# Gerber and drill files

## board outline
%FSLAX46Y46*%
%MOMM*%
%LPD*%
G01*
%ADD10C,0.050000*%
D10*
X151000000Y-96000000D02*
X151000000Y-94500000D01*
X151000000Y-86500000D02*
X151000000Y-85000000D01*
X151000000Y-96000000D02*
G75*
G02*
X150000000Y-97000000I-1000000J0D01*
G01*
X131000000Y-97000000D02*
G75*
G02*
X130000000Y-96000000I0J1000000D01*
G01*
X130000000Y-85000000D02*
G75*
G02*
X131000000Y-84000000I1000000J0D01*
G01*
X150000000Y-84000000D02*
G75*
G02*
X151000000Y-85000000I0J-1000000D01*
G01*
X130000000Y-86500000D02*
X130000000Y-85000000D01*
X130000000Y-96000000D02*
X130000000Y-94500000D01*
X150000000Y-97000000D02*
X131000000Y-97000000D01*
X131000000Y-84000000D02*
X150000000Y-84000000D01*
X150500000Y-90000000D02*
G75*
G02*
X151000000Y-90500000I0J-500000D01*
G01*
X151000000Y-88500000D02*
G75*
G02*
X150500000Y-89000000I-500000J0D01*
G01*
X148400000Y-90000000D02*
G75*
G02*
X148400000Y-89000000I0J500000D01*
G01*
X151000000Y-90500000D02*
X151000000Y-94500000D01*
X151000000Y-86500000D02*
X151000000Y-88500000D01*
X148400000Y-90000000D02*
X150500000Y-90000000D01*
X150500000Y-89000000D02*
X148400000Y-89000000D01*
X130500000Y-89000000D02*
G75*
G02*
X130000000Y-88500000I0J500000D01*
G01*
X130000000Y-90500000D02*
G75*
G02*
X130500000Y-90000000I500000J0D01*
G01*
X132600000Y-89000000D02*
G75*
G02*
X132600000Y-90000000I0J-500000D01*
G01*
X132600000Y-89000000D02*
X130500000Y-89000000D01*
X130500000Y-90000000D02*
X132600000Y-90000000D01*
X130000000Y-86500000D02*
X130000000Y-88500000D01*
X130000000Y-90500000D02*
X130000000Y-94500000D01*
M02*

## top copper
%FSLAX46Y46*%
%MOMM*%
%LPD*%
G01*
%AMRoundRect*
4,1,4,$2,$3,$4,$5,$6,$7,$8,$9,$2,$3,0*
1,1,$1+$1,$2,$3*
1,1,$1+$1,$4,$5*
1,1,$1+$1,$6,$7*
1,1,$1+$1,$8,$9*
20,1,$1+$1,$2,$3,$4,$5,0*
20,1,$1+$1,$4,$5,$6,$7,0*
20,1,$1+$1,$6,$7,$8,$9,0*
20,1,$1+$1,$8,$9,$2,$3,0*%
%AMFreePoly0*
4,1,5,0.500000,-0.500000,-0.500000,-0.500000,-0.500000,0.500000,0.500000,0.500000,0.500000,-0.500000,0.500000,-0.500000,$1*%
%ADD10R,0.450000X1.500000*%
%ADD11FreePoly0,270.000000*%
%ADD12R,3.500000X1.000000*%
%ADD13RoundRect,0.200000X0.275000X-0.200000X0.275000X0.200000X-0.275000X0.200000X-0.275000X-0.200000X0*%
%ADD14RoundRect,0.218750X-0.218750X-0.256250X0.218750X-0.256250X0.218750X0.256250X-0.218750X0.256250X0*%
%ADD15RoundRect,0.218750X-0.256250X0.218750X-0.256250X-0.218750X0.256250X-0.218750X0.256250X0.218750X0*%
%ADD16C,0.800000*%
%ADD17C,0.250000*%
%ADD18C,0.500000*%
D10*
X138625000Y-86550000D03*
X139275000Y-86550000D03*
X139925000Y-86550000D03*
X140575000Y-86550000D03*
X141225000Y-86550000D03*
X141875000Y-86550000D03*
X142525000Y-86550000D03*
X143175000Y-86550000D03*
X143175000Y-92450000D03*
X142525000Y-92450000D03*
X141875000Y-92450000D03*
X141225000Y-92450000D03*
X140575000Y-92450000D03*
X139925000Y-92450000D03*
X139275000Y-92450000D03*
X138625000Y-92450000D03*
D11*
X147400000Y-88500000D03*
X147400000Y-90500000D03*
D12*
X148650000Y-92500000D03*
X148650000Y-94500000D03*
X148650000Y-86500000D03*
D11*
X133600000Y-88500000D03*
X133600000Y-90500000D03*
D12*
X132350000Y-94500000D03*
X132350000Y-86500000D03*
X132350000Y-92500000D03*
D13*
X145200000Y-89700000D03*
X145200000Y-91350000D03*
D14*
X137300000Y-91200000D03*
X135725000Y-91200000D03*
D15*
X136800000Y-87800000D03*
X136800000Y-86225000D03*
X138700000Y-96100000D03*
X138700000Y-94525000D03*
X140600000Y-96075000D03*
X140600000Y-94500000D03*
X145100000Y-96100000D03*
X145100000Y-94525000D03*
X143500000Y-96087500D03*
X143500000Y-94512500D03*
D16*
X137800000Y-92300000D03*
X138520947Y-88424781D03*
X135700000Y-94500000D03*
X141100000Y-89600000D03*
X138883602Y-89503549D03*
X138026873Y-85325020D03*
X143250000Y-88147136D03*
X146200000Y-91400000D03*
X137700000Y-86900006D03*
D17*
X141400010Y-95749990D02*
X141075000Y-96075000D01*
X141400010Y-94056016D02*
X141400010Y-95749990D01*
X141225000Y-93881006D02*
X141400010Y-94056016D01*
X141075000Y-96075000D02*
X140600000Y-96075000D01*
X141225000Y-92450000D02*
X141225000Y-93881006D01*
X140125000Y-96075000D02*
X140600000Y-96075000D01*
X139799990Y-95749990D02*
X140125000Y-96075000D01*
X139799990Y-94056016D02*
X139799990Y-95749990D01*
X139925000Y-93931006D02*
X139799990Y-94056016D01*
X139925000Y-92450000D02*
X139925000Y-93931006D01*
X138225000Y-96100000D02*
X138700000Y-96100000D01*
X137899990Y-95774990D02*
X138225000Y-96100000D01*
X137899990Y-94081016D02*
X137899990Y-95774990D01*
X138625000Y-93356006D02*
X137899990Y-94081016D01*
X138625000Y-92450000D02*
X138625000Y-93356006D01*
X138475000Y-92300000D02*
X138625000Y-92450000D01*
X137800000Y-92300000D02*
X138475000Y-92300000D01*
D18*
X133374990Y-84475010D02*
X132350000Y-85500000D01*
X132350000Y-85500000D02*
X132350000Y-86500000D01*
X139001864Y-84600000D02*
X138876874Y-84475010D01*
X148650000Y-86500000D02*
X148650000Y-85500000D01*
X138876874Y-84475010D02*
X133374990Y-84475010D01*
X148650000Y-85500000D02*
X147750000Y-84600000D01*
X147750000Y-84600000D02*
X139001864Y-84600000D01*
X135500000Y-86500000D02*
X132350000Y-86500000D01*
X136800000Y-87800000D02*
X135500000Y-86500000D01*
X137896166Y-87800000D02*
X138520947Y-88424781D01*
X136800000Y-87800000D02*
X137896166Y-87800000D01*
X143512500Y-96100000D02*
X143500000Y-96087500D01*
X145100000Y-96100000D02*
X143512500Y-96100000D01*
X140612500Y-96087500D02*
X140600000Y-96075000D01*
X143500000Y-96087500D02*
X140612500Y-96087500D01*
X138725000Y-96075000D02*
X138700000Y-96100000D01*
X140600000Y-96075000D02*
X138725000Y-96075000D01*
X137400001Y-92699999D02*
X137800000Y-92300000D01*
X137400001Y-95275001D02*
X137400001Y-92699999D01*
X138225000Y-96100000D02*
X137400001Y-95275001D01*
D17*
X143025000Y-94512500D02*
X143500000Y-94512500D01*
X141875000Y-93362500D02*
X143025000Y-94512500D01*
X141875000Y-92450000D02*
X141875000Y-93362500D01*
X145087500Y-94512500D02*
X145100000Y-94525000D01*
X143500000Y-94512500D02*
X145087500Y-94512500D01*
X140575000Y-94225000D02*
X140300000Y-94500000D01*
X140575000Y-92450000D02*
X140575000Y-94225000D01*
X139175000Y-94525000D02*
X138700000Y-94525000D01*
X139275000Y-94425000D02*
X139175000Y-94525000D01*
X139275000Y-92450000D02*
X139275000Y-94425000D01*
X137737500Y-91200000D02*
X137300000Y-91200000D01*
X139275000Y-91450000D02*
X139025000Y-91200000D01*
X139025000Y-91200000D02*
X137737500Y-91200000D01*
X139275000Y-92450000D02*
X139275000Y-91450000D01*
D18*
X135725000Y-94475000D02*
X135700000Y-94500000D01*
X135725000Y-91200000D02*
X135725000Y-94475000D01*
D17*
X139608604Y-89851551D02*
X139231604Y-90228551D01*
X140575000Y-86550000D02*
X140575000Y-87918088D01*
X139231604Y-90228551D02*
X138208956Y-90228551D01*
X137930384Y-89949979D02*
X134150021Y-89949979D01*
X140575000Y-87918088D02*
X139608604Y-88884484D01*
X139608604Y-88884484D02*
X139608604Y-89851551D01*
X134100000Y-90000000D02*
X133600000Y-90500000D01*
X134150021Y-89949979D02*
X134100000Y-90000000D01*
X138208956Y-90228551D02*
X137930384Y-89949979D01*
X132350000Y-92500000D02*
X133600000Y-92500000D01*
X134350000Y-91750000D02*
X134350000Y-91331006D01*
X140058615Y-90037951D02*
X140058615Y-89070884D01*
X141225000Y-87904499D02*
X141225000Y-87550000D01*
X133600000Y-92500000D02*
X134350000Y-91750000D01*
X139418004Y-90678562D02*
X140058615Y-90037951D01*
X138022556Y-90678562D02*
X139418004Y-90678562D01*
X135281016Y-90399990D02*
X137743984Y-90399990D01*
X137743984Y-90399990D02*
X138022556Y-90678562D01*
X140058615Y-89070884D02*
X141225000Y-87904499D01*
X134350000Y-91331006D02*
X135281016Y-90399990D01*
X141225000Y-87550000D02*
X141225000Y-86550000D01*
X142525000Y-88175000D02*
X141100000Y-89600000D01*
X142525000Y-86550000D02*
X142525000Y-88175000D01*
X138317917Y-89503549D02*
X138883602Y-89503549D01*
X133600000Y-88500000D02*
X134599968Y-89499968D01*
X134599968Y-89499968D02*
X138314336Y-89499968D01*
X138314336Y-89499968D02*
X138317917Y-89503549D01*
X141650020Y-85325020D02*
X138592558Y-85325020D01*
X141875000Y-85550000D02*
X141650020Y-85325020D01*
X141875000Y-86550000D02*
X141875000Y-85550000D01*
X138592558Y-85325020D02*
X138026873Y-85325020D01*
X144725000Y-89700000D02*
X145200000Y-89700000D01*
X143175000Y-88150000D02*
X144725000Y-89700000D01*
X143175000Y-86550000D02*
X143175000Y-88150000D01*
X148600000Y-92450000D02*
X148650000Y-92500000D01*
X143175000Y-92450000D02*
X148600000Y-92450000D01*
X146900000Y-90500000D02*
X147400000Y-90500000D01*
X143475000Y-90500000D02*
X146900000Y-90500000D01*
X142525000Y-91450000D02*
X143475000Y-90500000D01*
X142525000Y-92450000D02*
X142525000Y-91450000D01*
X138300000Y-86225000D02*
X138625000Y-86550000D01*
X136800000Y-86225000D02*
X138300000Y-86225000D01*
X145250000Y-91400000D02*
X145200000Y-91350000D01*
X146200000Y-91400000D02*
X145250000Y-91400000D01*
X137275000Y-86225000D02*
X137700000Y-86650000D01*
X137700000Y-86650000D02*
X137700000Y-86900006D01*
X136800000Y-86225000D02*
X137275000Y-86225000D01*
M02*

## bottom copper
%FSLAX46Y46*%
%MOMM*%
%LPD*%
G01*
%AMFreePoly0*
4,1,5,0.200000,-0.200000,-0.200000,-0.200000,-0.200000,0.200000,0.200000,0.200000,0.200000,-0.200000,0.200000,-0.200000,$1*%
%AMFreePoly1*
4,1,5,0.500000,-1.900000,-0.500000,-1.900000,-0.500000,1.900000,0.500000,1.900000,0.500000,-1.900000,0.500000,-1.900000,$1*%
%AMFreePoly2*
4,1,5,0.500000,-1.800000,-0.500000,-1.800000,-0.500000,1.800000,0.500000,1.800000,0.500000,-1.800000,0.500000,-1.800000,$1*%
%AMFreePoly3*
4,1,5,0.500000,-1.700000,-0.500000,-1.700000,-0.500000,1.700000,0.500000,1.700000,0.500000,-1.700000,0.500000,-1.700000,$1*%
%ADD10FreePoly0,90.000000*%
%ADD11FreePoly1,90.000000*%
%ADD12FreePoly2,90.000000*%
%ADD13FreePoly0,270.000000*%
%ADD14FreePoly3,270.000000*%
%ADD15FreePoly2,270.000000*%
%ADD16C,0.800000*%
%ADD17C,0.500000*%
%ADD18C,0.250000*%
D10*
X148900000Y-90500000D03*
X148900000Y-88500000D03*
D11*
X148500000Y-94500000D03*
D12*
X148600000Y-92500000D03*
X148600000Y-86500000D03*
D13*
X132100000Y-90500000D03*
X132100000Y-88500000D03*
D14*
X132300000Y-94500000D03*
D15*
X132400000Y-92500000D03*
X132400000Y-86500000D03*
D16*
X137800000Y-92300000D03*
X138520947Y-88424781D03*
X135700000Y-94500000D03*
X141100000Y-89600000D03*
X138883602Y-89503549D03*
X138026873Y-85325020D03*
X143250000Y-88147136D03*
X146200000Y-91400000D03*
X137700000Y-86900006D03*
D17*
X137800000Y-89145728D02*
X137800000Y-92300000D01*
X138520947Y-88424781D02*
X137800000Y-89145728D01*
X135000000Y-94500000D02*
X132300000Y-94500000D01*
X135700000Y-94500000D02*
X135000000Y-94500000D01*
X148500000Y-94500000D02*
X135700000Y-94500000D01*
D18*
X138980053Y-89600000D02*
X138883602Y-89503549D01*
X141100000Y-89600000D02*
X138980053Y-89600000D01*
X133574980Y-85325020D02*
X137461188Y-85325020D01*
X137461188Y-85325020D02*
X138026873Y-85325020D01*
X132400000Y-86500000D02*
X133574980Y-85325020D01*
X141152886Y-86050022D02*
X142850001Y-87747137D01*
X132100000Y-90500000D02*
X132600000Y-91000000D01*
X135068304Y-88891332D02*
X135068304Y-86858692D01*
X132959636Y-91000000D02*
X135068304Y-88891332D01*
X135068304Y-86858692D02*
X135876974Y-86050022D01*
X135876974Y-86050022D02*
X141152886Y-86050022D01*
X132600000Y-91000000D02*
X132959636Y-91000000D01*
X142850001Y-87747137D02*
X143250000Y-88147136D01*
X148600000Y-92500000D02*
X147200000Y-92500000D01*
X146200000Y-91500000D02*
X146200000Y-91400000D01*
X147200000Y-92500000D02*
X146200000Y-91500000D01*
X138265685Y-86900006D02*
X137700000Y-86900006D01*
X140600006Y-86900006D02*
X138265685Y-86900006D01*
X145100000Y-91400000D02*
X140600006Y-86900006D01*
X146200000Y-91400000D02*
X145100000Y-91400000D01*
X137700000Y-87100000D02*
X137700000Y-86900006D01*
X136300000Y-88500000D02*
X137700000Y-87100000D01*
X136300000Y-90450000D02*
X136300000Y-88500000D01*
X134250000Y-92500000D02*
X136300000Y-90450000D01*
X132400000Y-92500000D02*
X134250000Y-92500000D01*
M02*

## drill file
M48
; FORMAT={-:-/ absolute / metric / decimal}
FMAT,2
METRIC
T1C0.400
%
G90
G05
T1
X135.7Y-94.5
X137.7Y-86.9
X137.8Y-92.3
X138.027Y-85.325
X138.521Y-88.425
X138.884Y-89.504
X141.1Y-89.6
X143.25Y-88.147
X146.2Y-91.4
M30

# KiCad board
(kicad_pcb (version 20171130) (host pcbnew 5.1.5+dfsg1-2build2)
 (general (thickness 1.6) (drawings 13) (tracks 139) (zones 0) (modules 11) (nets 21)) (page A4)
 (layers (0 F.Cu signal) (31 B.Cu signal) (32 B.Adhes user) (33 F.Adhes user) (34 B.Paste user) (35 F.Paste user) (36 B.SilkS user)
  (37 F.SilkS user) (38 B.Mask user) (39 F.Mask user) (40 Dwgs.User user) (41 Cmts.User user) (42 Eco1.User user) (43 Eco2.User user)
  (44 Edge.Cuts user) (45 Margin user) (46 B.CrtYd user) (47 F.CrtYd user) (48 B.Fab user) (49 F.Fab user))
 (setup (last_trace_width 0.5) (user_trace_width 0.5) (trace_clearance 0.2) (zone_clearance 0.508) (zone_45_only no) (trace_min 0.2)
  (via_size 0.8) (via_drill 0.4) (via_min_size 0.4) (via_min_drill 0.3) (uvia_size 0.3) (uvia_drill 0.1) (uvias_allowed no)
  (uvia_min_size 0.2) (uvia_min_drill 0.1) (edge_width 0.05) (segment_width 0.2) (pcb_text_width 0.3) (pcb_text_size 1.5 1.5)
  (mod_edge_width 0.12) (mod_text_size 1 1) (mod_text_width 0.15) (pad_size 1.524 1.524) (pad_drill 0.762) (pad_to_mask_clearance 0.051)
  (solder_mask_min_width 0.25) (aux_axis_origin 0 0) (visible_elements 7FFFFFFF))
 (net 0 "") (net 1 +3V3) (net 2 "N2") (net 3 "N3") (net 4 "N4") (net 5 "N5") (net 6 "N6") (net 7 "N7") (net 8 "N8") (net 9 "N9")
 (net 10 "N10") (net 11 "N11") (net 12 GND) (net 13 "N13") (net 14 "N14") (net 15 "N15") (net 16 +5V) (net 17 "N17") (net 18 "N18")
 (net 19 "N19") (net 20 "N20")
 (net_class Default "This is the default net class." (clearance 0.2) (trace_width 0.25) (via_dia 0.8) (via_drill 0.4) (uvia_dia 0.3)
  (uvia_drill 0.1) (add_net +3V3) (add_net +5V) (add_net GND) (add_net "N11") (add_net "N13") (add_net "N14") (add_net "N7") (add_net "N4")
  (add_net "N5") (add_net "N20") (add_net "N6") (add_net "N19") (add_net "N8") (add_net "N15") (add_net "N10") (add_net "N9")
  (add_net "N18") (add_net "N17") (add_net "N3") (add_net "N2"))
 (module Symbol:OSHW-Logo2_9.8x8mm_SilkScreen (layer B.Cu) (at 141 90 180)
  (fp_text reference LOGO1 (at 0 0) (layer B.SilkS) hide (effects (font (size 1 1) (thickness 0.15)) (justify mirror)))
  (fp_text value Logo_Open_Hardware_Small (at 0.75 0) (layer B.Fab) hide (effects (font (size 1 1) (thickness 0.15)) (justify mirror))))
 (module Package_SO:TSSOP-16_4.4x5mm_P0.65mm (layer F.Cu) (at 140.9 89.5 90)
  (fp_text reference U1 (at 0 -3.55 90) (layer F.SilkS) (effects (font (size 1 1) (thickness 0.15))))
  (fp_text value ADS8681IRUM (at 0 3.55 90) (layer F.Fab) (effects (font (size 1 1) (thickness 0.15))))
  (pad 16 smd rect (at 2.95 -2.275 90) (size 1.5 0.45) (layers F.Cu F.Paste F.Mask) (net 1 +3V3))
  (pad 15 smd rect (at 2.95 -1.625 90) (size 1.5 0.45) (layers F.Cu F.Paste F.Mask) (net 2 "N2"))
  (pad 14 smd rect (at 2.95 -0.975 90) (size 1.5 0.45) (layers F.Cu F.Paste F.Mask) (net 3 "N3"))
  (pad 13 smd rect (at 2.95 -0.325 90) (size 1.5 0.45) (layers F.Cu F.Paste F.Mask) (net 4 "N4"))
  (pad 12 smd rect (at 2.95 0.325 90) (size 1.5 0.45) (layers F.Cu F.Paste F.Mask) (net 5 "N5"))
  (pad 11 smd rect (at 2.95 0.975 90) (size 1.5 0.45) (layers F.Cu F.Paste F.Mask) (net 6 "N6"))
  (pad 10 smd rect (at 2.95 1.625 90) (size 1.5 0.45) (layers F.Cu F.Paste F.Mask) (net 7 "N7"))
  (pad 9 smd rect (at 2.95 2.275 90) (size 1.5 0.45) (layers F.Cu F.Paste F.Mask) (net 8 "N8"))
  (pad 8 smd rect (at -2.95 2.275 90) (size 1.5 0.45) (layers F.Cu F.Paste F.Mask) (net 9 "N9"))
  (pad 7 smd rect (at -2.95 1.625 90) (size 1.5 0.45) (layers F.Cu F.Paste F.Mask) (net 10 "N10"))
  (pad 6 smd rect (at -2.95 0.975 90) (size 1.5 0.45) (layers F.Cu F.Paste F.Mask) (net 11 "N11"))
  (pad 5 smd rect (at -2.95 0.325 90) (size 1.5 0.45) (layers F.Cu F.Paste F.Mask) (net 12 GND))
  (pad 4 smd rect (at -2.95 -0.325 90) (size 1.5 0.45) (layers F.Cu F.Paste F.Mask) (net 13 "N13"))
  (pad 3 smd rect (at -2.95 -0.975 90) (size 1.5 0.45) (layers F.Cu F.Paste F.Mask) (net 12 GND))
  (pad 2 smd rect (at -2.95 -1.625 90) (size 1.5 0.45) (layers F.Cu F.Paste F.Mask) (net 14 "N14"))
  (pad 1 smd rect (at -2.95 -2.275 90) (size 1.5 0.45) (layers F.Cu F.Paste F.Mask) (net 12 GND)))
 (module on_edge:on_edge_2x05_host (layer F.Cu) (at 151 90.5 270)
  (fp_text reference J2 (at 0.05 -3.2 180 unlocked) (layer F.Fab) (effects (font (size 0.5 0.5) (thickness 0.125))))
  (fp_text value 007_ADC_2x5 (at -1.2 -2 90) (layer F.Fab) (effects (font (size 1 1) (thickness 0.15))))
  (fp_arc (start 0 0.5) (end 0 0) (angle -90) (layer Edge.Cuts) (width 0.05))
  (fp_arc (start -2 0.5) (end -1.5 0.5) (angle -90) (layer Edge.Cuts) (width 0.05))
  (fp_arc (start -1 2.6) (end -1.5 2.6) (angle -180) (layer Edge.Cuts) (width 0.05))
  (fp_line (start 0 0) (end 4 0) (layer Edge.Cuts) (width 0.05))
  (fp_line (start -4 0) (end -2 0) (layer Edge.Cuts) (width 0.05))
  (fp_line (start -0.5 2.6) (end -0.5 0.5) (layer Edge.Cuts) (width 0.05))
  (fp_line (start -1.5 0.5) (end -1.5 2.6) (layer Edge.Cuts) (width 0.05))
  (pad 2 smd custom (at -2 3.6 270) (size 1 1) (layers F.Cu F.Mask) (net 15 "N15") (zone_connect 0)
   (options (clearance outline) (anchor rect)) (primitives))
  (pad 3 smd custom (at 0 3.6 270) (size 1 1) (layers F.Cu F.Mask) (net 10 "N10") (zone_connect 0)
   (options (clearance outline) (anchor rect)) (primitives))
  (pad 8 smd custom (at 0 2.1 90) (size 0.4 0.4) (layers B.Cu B.Mask) (zone_connect 0) (options (clearance outline) (anchor rect))
   (primitives))
  (pad 7 smd custom (at -2 2.1 90) (size 0.4 0.4) (layers B.Cu B.Mask) (zone_connect 0) (options (clearance outline) (anchor rect))
   (primitives))
  (pad 4 smd rect (at 2 2.35 270) (size 1 3.5) (layers F.Cu F.Mask) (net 9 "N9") (zone_connect 0))
  (pad 10 smd custom (at 4 2.5 90) (size 1 3.8) (layers B.Cu B.Mask) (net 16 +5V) (zone_connect 0)
   (options (clearance outline) (anchor rect)) (primitives))
  (pad 9 smd custom (at 2 2.4 90) (size 1 3.6) (layers B.Cu B.Mask) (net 1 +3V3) (zone_connect 0)
   (options (clearance outline) (anchor rect)) (primitives))
  (pad 6 smd custom (at -4 2.4 90) (size 1 3.6) (layers B.Cu B.Mask) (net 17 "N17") (zone_connect 0)
   (options (clearance outline) (anchor rect)) (primitives))
  (pad 5 smd rect (at 4 2.35 270) (size 1 3.5) (layers F.Cu F.Mask) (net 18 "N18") (zone_connect 0))
  (pad 1 smd rect (at -4 2.35 270) (size 1 3.5) (layers F.Cu F.Mask) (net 12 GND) (zone_connect 0)))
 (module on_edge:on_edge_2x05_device (layer F.Cu) (at 130 90.5 270)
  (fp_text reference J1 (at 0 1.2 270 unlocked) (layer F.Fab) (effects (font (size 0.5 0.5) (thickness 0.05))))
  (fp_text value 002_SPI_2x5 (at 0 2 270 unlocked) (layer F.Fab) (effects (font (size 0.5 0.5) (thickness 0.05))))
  (fp_arc (start -2 -0.5) (end -2 0) (angle -90) (layer Edge.Cuts) (width 0.05))
  (fp_arc (start 0 -0.5) (end -0.5 -0.5) (angle -90) (layer Edge.Cuts) (width 0.05))
  (fp_arc (start -1 -2.6) (end -0.5 -2.6) (angle -180) (layer Edge.Cuts) (width 0.05))
  (fp_line (start -1.5 -2.6) (end -1.5 -0.5) (layer Edge.Cuts) (width 0.05))
  (fp_line (start -0.5 -0.5) (end -0.5 -2.6) (layer Edge.Cuts) (width 0.05))
  (fp_line (start -4 0) (end -2 0) (layer Edge.Cuts) (width 0.05))
  (fp_line (start 0 0) (end 4 0) (layer Edge.Cuts) (width 0.05))
  (pad 2 smd custom (at -2 -3.6 270) (size 1 1) (layers F.Cu F.Mask) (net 7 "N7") (zone_connect 0)
   (options (clearance outline) (anchor rect)) (primitives))
  (pad 3 smd custom (at 0 -3.6 270) (size 1 1) (layers F.Cu F.Mask) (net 4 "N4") (zone_connect 0)
   (options (clearance outline) (anchor rect)) (primitives))
  (pad 8 smd custom (at 0 -2.1 270) (size 0.4 0.4) (layers B.Cu B.Mask) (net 8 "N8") (zone_connect 0)
   (options (clearance outline) (anchor rect)) (primitives))
  (pad 7 smd custom (at -2 -2.1 270) (size 0.4 0.4) (layers B.Cu B.Mask) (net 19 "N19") (zone_connect 0)
   (options (clearance outline) (anchor rect)) (primitives))
  (pad 10 smd custom (at 4 -2.3 270) (size 1 3.4) (layers B.Cu B.Mask) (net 16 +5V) (zone_connect 0)
   (options (clearance outline) (anchor rect)) (primitives))
  (pad 9 smd custom (at 2 -2.4 270) (size 1 3.6) (layers B.Cu B.Mask) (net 1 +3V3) (zone_connect 0)
   (options (clearance outline) (anchor rect)) (primitives))
  (pad 6 smd custom (at -4 -2.4 270) (size 1 3.6) (layers B.Cu B.Mask) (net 6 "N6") (zone_connect 0)
   (options (clearance outline) (anchor rect)) (primitives))
  (pad 5 smd rect (at 4 -2.35 90) (size 1 3.5) (layers F.Cu F.Mask) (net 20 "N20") (zone_connect 0))
  (pad 1 smd rect (at -4 -2.35 90) (size 1 3.5) (layers F.Cu F.Mask) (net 12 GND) (zone_connect 0))
  (pad 4 smd rect (at 2 -2.35 90) (size 1 3.5) (layers F.Cu F.Mask) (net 5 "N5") (zone_connect 0)))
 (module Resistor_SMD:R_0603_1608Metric (layer F.Cu) (at 145.2 90.525 90)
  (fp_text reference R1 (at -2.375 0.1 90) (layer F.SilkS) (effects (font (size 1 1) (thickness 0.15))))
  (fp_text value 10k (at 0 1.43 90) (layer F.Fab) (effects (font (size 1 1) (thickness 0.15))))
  (pad 2 smd roundrect (at 0.825 0 90) (size 0.8 0.95) (layers F.Cu F.Paste F.Mask) (roundrect_rratio 0.25) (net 8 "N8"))
  (pad 1 smd roundrect (at -0.825 0 90) (size 0.8 0.95) (layers F.Cu F.Paste F.Mask) (roundrect_rratio 0.25) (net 1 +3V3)))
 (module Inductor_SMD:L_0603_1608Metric (layer F.Cu) (at 136.5125 91.2)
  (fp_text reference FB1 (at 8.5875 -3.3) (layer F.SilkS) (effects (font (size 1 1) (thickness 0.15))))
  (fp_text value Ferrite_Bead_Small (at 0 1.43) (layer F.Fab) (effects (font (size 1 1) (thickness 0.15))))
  (pad 2 smd roundrect (at 0.7875 0) (size 0.875 0.95) (layers F.Cu F.Paste F.Mask) (roundrect_rratio 0.25) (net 14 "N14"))
  (pad 1 smd roundrect (at -0.7875 0) (size 0.875 0.95) (layers F.Cu F.Paste F.Mask) (roundrect_rratio 0.25) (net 16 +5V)))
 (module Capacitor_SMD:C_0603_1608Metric (layer F.Cu) (at 136.8 87.0125 270)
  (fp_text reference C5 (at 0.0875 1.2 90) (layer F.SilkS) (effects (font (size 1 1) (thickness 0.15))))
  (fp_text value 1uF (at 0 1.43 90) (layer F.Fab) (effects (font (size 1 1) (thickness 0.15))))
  (pad 2 smd roundrect (at 0.7875 0 270) (size 0.875 0.95) (layers F.Cu F.Paste F.Mask) (roundrect_rratio 0.25) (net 12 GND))
  (pad 1 smd roundrect (at -0.7875 0 270) (size 0.875 0.95) (layers F.Cu F.Paste F.Mask) (roundrect_rratio 0.25) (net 1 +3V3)))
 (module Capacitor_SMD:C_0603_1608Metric (layer F.Cu) (at 138.7 95.3125 270)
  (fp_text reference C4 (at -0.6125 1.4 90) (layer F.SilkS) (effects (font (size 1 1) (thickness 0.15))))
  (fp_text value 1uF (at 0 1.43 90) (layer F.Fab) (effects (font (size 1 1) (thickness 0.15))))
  (pad 2 smd roundrect (at 0.7875 0 270) (size 0.875 0.95) (layers F.Cu F.Paste F.Mask) (roundrect_rratio 0.25) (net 12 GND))
  (pad 1 smd roundrect (at -0.7875 0 270) (size 0.875 0.95) (layers F.Cu F.Paste F.Mask) (roundrect_rratio 0.25) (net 14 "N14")))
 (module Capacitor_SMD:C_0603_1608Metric (layer F.Cu) (at 140.6 95.2875 270)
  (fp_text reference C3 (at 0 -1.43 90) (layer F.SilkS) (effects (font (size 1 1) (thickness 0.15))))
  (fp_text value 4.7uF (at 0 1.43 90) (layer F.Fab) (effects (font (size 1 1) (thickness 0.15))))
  (pad 2 smd roundrect (at 0.7875 0 270) (size 0.875 0.95) (layers F.Cu F.Paste F.Mask) (roundrect_rratio 0.25) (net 12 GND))
  (pad 1 smd roundrect (at -0.7875 0 270) (size 0.875 0.95) (layers F.Cu F.Paste F.Mask) (roundrect_rratio 0.25) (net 13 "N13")))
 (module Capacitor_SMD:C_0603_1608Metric (layer F.Cu) (at 145.1 95.3125 270)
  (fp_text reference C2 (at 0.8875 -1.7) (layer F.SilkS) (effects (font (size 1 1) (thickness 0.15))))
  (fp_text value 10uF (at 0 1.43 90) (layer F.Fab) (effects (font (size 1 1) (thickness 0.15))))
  (pad 2 smd roundrect (at 0.7875 0 270) (size 0.875 0.95) (layers F.Cu F.Paste F.Mask) (roundrect_rratio 0.25) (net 12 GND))
  (pad 1 smd roundrect (at -0.7875 0 270) (size 0.875 0.95) (layers F.Cu F.Paste F.Mask) (roundrect_rratio 0.25) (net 11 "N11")))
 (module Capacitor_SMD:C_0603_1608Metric (layer F.Cu) (at 143.5 95.3 270)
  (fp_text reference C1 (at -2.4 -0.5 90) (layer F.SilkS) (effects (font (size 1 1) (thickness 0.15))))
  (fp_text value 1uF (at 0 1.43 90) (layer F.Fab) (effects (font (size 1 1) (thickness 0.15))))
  (pad 2 smd roundrect (at 0.7875 0 270) (size 0.875 0.95) (layers F.Cu F.Paste F.Mask) (roundrect_rratio 0.25) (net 12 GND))
  (pad 1 smd roundrect (at -0.7875 0 270) (size 0.875 0.95) (layers F.Cu F.Paste F.Mask) (roundrect_rratio 0.25) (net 11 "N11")))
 (gr_line (start 151 96) (end 151 94.5) (layer Edge.Cuts) (width 0.05))
 (gr_line (start 151 86.5) (end 151 85) (layer Edge.Cuts) (width 0.05))
 (gr_arc (start 150 96) (end 150 97) (angle -90) (layer Edge.Cuts) (width 0.05))
 (gr_arc (start 131 96) (end 130 96) (angle -90) (layer Edge.Cuts) (width 0.05))
 (gr_arc (start 131 85) (end 131 84) (angle -90) (layer Edge.Cuts) (width 0.05))
 (gr_arc (start 150 85) (end 151 85) (angle -90) (layer Edge.Cuts) (width 0.05))
 (gr_line (start 130 86.5) (end 130 85) (layer Edge.Cuts) (width 0.05))
 (gr_line (start 130 96) (end 130 94.5) (layer Edge.Cuts) (width 0.05))
 (gr_line (start 150 97) (end 131 97) (layer Edge.Cuts) (width 0.05))
 (gr_line (start 131 84) (end 150 84) (layer Edge.Cuts) (width 0.05))
 (segment (start 141.40001 95.74999) (end 141.075 96.075) (width 0.25) (layer F.Cu) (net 12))
 (segment (start 141.40001 94.056016) (end 141.40001 95.74999) (width 0.25) (layer F.Cu) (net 12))
 (segment (start 141.225 93.881006) (end 141.40001 94.056016) (width 0.25) (layer F.Cu) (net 12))
 (segment (start 141.075 96.075) (end 140.6 96.075) (width 0.25) (layer F.Cu) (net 12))
 (segment (start 141.225 92.45) (end 141.225 93.881006) (width 0.25) (layer F.Cu) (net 12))
 (segment (start 140.125 96.075) (end 140.6 96.075) (width 0.25) (layer F.Cu) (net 12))
 (segment (start 139.79999 95.74999) (end 140.125 96.075) (width 0.25) (layer F.Cu) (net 12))
 (segment (start 139.79999 94.056016) (end 139.79999 95.74999) (width 0.25) (layer F.Cu) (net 12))
 (segment (start 139.925 93.931006) (end 139.79999 94.056016) (width 0.25) (layer F.Cu) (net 12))
 (segment (start 139.925 92.45) (end 139.925 93.931006) (width 0.25) (layer F.Cu) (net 12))
 (segment (start 138.225 96.1) (end 138.7 96.1) (width 0.25) (layer F.Cu) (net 12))
 (segment (start 137.89999 95.77499) (end 138.225 96.1) (width 0.25) (layer F.Cu) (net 12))
 (segment (start 137.89999 94.081016) (end 137.89999 95.77499) (width 0.25) (layer F.Cu) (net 12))
 (segment (start 138.625 93.356006) (end 137.89999 94.081016) (width 0.25) (layer F.Cu) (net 12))
 (segment (start 138.625 92.45) (end 138.625 93.356006) (width 0.25) (layer F.Cu) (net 12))
 (via (at 137.8 92.3) (size 0.8) (drill 0.4) (layers F.Cu B.Cu) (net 12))
 (segment (start 138.475 92.3) (end 138.625 92.45) (width 0.25) (layer F.Cu) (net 12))
 (segment (start 137.8 92.3) (end 138.475 92.3) (width 0.25) (layer F.Cu) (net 12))
 (segment (start 133.37499 84.47501) (end 132.35 85.5) (width 0.5) (layer F.Cu) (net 12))
 (via (at 138.520947 88.424781) (size 0.8) (drill 0.4) (layers F.Cu B.Cu) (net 12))
 (segment (start 132.35 85.5) (end 132.35 86.5) (width 0.5) (layer F.Cu) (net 12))
 (segment (start 139.001864 84.6) (end 138.876874 84.47501) (width 0.5) (layer F.Cu) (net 12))
 (segment (start 148.65 86.5) (end 148.65 85.5) (width 0.5) (layer F.Cu) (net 12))
 (segment (start 138.876874 84.47501) (end 133.37499 84.47501) (width 0.5) (layer F.Cu) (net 12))
 (segment (start 148.65 85.5) (end 147.75 84.6) (width 0.5) (layer F.Cu) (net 12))
 (segment (start 147.75 84.6) (end 139.001864 84.6) (width 0.5) (layer F.Cu) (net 12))
 (segment (start 135.5 86.5) (end 132.35 86.5) (width 0.5) (layer F.Cu) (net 12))
 (segment (start 136.8 87.8) (end 135.5 86.5) (width 0.5) (layer F.Cu) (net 12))
 (segment (start 137.896166 87.8) (end 138.520947 88.424781) (width 0.5) (layer F.Cu) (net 12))
 (segment (start 136.8 87.8) (end 137.896166 87.8) (width 0.5) (layer F.Cu) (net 12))
 (segment (start 137.8 89.145728) (end 137.8 92.3) (width 0.5) (layer B.Cu) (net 12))
 (segment (start 138.520947 88.424781) (end 137.8 89.145728) (width 0.5) (layer B.Cu) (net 12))
 (segment (start 143.5125 96.1) (end 143.5 96.0875) (width 0.5) (layer F.Cu) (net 12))
 (segment (start 145.1 96.1) (end 143.5125 96.1) (width 0.5) (layer F.Cu) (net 12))
 (segment (start 140.6125 96.0875) (end 140.6 96.075) (width 0.5) (layer F.Cu) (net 12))
 (segment (start 143.5 96.0875) (end 140.6125 96.0875) (width 0.5) (layer F.Cu) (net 12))
 (segment (start 138.725 96.075) (end 138.7 96.1) (width 0.5) (layer F.Cu) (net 12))
 (segment (start 140.6 96.075) (end 138.725 96.075) (width 0.5) (layer F.Cu) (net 12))
 (segment (start 137.400001 92.699999) (end 137.8 92.3) (width 0.5) (layer F.Cu) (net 12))
 (segment (start 137.400001 95.275001) (end 137.400001 92.699999) (width 0.5) (layer F.Cu) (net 12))
 (segment (start 138.225 96.1) (end 137.400001 95.275001) (width 0.5) (layer F.Cu) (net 12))
 (segment (start 143.025 94.5125) (end 143.5 94.5125) (width 0.25) (layer F.Cu) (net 11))
 (segment (start 141.875 93.3625) (end 143.025 94.5125) (width 0.25) (layer F.Cu) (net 11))
 (segment (start 141.875 92.45) (end 141.875 93.3625) (width 0.25) (layer F.Cu) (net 11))
 (segment (start 145.0875 94.5125) (end 145.1 94.525) (width 0.25) (layer F.Cu) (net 11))
 (segment (start 143.5 94.5125) (end 145.0875 94.5125) (width 0.25) (layer F.Cu) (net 11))
 (segment (start 140.575 94.225) (end 140.3 94.5) (width 0.25) (layer F.Cu) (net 13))
 (segment (start 140.575 92.45) (end 140.575 94.225) (width 0.25) (layer F.Cu) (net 13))
 (segment (start 139.175 94.525) (end 138.7 94.525) (width 0.25) (layer F.Cu) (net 14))
 (segment (start 139.275 94.425) (end 139.175 94.525) (width 0.25) (layer F.Cu) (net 14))
 (segment (start 139.275 92.45) (end 139.275 94.425) (width 0.25) (layer F.Cu) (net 14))
 (segment (start 137.7375 91.2) (end 137.3 91.2) (width 0.25) (layer F.Cu) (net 14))
 (segment (start 139.275 91.45) (end 139.025 91.2) (width 0.25) (layer F.Cu) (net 14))
 (segment (start 139.025 91.2) (end 137.7375 91.2) (width 0.25) (layer F.Cu) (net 14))
 (segment (start 139.275 92.45) (end 139.275 91.45) (width 0.25) (layer F.Cu) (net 14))
 (segment (start 135 94.5) (end 132.3 94.5) (width 0.5) (layer B.Cu) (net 16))
 (segment (start 135.725 94.475) (end 135.7 94.5) (width 0.5) (layer F.Cu) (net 16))
 (segment (start 135.725 91.2) (end 135.725 94.475) (width 0.5) (layer F.Cu) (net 16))
 (segment (start 135.7 94.5) (end 135 94.5) (width 0.5) (layer B.Cu) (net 16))
 (via (at 135.7 94.5) (size 0.8) (drill 0.4) (layers F.Cu B.Cu) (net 16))
 (segment (start 148.5 94.5) (end 135.7 94.5) (width 0.5) (layer B.Cu) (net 16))
 (segment (start 139.608604 89.851551) (end 139.231604 90.228551) (width 0.25) (layer F.Cu) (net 4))
 (segment (start 140.575 86.55) (end 140.575 87.918088) (width 0.25) (layer F.Cu) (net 4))
 (segment (start 139.231604 90.228551) (end 138.208956 90.228551) (width 0.25) (layer F.Cu) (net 4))
 (segment (start 137.930384 89.949979) (end 134.150021 89.949979) (width 0.25) (layer F.Cu) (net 4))
 (segment (start 140.575 87.918088) (end 139.608604 88.884484) (width 0.25) (layer F.Cu) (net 4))
 (segment (start 139.608604 88.884484) (end 139.608604 89.851551) (width 0.25) (layer F.Cu) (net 4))
 (segment (start 134.1 90) (end 133.6 90.5) (width 0.25) (layer F.Cu) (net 4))
 (segment (start 134.150021 89.949979) (end 134.1 90) (width 0.25) (layer F.Cu) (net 4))
 (segment (start 138.208956 90.228551) (end 137.930384 89.949979) (width 0.25) (layer F.Cu) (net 4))
 (segment (start 132.35 92.5) (end 133.6 92.5) (width 0.25) (layer F.Cu) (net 5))
 (segment (start 134.35 91.75) (end 134.35 91.331006) (width 0.25) (layer F.Cu) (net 5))
 (segment (start 140.058615 90.037951) (end 140.058615 89.070884) (width 0.25) (layer F.Cu) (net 5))
 (segment (start 141.225 87.904499) (end 141.225 87.55) (width 0.25) (layer F.Cu) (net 5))
 (segment (start 133.6 92.5) (end 134.35 91.75) (width 0.25) (layer F.Cu) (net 5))
 (segment (start 139.418004 90.678562) (end 140.058615 90.037951) (width 0.25) (layer F.Cu) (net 5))
 (segment (start 138.022556 90.678562) (end 139.418004 90.678562) (width 0.25) (layer F.Cu) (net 5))
 (segment (start 135.281016 90.39999) (end 137.743984 90.39999) (width 0.25) (layer F.Cu) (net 5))
 (segment (start 137.743984 90.39999) (end 138.022556 90.678562) (width 0.25) (layer F.Cu) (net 5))
 (segment (start 140.058615 89.070884) (end 141.225 87.904499) (width 0.25) (layer F.Cu) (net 5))
 (segment (start 134.35 91.331006) (end 135.281016 90.39999) (width 0.25) (layer F.Cu) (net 5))
 (segment (start 141.225 87.55) (end 141.225 86.55) (width 0.25) (layer F.Cu) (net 5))
 (via (at 141.1 89.6) (size 0.8) (drill 0.4) (layers F.Cu B.Cu) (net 7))
 (segment (start 142.525 88.175) (end 141.1 89.6) (width 0.25) (layer F.Cu) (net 7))
 (segment (start 142.525 86.55) (end 142.525 88.175) (width 0.25) (layer F.Cu) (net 7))
 (segment (start 138.317917 89.503549) (end 138.883602 89.503549) (width 0.25) (layer F.Cu) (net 7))
 (segment (start 133.6 88.5) (end 134.599968 89.499968) (width 0.25) (layer F.Cu) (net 7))
 (segment (start 134.599968 89.499968) (end 138.314336 89.499968) (width 0.25) (layer F.Cu) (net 7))
 (via (at 138.883602 89.503549) (size 0.8) (drill 0.4) (layers F.Cu B.Cu) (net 7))
 (segment (start 138.314336 89.499968) (end 138.317917 89.503549) (width 0.25) (layer F.Cu) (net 7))
 (segment (start 138.980053 89.6) (end 138.883602 89.503549) (width 0.25) (layer B.Cu) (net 7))
 (segment (start 141.1 89.6) (end 138.980053 89.6) (width 0.25) (layer B.Cu) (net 7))
 (segment (start 141.65002 85.32502) (end 138.592558 85.32502) (width 0.25) (layer F.Cu) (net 6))
 (segment (start 141.875 85.55) (end 141.65002 85.32502) (width 0.25) (layer F.Cu) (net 6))
 (via (at 138.026873 85.32502) (size 0.8) (drill 0.4) (layers F.Cu B.Cu) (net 6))
 (segment (start 141.875 86.55) (end 141.875 85.55) (width 0.25) (layer F.Cu) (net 6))
 (segment (start 133.57498 85.32502) (end 137.461188 85.32502) (width 0.25) (layer B.Cu) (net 6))
 (segment (start 137.461188 85.32502) (end 138.026873 85.32502) (width 0.25) (layer B.Cu) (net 6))
 (segment (start 132.4 86.5) (end 133.57498 85.32502) (width 0.25) (layer B.Cu) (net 6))
 (segment (start 138.592558 85.32502) (end 138.026873 85.32502) (width 0.25) (layer F.Cu) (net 6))
 (segment (start 144.725 89.7) (end 145.2 89.7) (width 0.25) (layer F.Cu) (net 8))
 (segment (start 143.175 88.15) (end 144.725 89.7) (width 0.25) (layer F.Cu) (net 8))
 (segment (start 143.175 86.55) (end 143.175 88.15) (width 0.25) (layer F.Cu) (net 8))
 (via (at 143.25 88.147136) (size 0.8) (drill 0.4) (layers F.Cu B.Cu) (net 8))
 (segment (start 141.152886 86.050022) (end 142.850001 87.747137) (width 0.25) (layer B.Cu) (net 8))
 (segment (start 132.1 90.5) (end 132.6 91) (width 0.25) (layer B.Cu) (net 8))
 (segment (start 135.068304 88.891332) (end 135.068304 86.858692) (width 0.25) (layer B.Cu) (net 8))
 (segment (start 132.959636 91) (end 135.068304 88.891332) (width 0.25) (layer B.Cu) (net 8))
 (segment (start 135.068304 86.858692) (end 135.876974 86.050022) (width 0.25) (layer B.Cu) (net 8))
 (segment (start 135.876974 86.050022) (end 141.152886 86.050022) (width 0.25) (layer B.Cu) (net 8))
 (segment (start 132.6 91) (end 132.959636 91) (width 0.25) (layer B.Cu) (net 8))
 (segment (start 142.850001 87.747137) (end 143.25 88.147136) (width 0.25) (layer B.Cu) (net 8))
 (segment (start 148.6 92.45) (end 148.65 92.5) (width 0.25) (layer F.Cu) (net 9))
 (segment (start 143.175 92.45) (end 148.6 92.45) (width 0.25) (layer F.Cu) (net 9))
 (segment (start 146.9 90.5) (end 147.4 90.5) (width 0.25) (layer F.Cu) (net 10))
 (segment (start 143.475 90.5) (end 146.9 90.5) (width 0.25) (layer F.Cu) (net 10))
 (segment (start 142.525 91.45) (end 143.475 90.5) (width 0.25) (layer F.Cu) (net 10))
 (segment (start 142.525 92.45) (end 142.525 91.45) (width 0.25) (layer F.Cu) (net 10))
 (segment (start 138.3 86.225) (end 138.625 86.55) (width 0.25) (layer F.Cu) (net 1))
 (segment (start 136.8 86.225) (end 138.3 86.225) (width 0.25) (layer F.Cu) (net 1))
 (segment (start 148.6 92.5) (end 147.2 92.5) (width 0.25) (layer B.Cu) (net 1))
 (via (at 146.2 91.4) (size 0.8) (drill 0.4) (layers F.Cu B.Cu) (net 1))
 (segment (start 146.2 91.5) (end 146.2 91.4) (width 0.25) (layer B.Cu) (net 1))
 (segment (start 147.2 92.5) (end 146.2 91.5) (width 0.25) (layer B.Cu) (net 1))
 (segment (start 145.25 91.4) (end 145.2 91.35) (width 0.25) (layer F.Cu) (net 1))
 (segment (start 146.2 91.4) (end 145.25 91.4) (width 0.25) (layer F.Cu) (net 1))
 (segment (start 137.275 86.225) (end 137.7 86.65) (width 0.25) (layer F.Cu) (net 1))
 (segment (start 137.7 86.65) (end 137.7 86.900006) (width 0.25) (layer F.Cu) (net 1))
 (segment (start 138.265685 86.900006) (end 137.7 86.900006) (width 0.25) (layer B.Cu) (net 1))
 (segment (start 140.600006 86.900006) (end 138.265685 86.900006) (width 0.25) (layer B.Cu) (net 1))
 (segment (start 145.1 91.4) (end 140.600006 86.900006) (width 0.25) (layer B.Cu) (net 1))
 (via (at 137.7 86.900006) (size 0.8) (drill 0.4) (layers F.Cu B.Cu) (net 1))
 (segment (start 136.8 86.225) (end 137.275 86.225) (width 0.25) (layer F.Cu) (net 1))
 (segment (start 146.2 91.4) (end 145.1 91.4) (width 0.25) (layer B.Cu) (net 1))
 (segment (start 137.7 87.1) (end 137.7 86.900006) (width 0.25) (layer B.Cu) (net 1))
 (segment (start 136.3 88.5) (end 137.7 87.1) (width 0.25) (layer B.Cu) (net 1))
 (segment (start 136.3 90.45) (end 136.3 88.5) (width 0.25) (layer B.Cu) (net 1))
 (segment (start 134.25 92.5) (end 136.3 90.45) (width 0.25) (layer B.Cu) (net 1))
 (segment (start 132.4 92.5) (end 134.25 92.5) (width 0.25) (layer B.Cu) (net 1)))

